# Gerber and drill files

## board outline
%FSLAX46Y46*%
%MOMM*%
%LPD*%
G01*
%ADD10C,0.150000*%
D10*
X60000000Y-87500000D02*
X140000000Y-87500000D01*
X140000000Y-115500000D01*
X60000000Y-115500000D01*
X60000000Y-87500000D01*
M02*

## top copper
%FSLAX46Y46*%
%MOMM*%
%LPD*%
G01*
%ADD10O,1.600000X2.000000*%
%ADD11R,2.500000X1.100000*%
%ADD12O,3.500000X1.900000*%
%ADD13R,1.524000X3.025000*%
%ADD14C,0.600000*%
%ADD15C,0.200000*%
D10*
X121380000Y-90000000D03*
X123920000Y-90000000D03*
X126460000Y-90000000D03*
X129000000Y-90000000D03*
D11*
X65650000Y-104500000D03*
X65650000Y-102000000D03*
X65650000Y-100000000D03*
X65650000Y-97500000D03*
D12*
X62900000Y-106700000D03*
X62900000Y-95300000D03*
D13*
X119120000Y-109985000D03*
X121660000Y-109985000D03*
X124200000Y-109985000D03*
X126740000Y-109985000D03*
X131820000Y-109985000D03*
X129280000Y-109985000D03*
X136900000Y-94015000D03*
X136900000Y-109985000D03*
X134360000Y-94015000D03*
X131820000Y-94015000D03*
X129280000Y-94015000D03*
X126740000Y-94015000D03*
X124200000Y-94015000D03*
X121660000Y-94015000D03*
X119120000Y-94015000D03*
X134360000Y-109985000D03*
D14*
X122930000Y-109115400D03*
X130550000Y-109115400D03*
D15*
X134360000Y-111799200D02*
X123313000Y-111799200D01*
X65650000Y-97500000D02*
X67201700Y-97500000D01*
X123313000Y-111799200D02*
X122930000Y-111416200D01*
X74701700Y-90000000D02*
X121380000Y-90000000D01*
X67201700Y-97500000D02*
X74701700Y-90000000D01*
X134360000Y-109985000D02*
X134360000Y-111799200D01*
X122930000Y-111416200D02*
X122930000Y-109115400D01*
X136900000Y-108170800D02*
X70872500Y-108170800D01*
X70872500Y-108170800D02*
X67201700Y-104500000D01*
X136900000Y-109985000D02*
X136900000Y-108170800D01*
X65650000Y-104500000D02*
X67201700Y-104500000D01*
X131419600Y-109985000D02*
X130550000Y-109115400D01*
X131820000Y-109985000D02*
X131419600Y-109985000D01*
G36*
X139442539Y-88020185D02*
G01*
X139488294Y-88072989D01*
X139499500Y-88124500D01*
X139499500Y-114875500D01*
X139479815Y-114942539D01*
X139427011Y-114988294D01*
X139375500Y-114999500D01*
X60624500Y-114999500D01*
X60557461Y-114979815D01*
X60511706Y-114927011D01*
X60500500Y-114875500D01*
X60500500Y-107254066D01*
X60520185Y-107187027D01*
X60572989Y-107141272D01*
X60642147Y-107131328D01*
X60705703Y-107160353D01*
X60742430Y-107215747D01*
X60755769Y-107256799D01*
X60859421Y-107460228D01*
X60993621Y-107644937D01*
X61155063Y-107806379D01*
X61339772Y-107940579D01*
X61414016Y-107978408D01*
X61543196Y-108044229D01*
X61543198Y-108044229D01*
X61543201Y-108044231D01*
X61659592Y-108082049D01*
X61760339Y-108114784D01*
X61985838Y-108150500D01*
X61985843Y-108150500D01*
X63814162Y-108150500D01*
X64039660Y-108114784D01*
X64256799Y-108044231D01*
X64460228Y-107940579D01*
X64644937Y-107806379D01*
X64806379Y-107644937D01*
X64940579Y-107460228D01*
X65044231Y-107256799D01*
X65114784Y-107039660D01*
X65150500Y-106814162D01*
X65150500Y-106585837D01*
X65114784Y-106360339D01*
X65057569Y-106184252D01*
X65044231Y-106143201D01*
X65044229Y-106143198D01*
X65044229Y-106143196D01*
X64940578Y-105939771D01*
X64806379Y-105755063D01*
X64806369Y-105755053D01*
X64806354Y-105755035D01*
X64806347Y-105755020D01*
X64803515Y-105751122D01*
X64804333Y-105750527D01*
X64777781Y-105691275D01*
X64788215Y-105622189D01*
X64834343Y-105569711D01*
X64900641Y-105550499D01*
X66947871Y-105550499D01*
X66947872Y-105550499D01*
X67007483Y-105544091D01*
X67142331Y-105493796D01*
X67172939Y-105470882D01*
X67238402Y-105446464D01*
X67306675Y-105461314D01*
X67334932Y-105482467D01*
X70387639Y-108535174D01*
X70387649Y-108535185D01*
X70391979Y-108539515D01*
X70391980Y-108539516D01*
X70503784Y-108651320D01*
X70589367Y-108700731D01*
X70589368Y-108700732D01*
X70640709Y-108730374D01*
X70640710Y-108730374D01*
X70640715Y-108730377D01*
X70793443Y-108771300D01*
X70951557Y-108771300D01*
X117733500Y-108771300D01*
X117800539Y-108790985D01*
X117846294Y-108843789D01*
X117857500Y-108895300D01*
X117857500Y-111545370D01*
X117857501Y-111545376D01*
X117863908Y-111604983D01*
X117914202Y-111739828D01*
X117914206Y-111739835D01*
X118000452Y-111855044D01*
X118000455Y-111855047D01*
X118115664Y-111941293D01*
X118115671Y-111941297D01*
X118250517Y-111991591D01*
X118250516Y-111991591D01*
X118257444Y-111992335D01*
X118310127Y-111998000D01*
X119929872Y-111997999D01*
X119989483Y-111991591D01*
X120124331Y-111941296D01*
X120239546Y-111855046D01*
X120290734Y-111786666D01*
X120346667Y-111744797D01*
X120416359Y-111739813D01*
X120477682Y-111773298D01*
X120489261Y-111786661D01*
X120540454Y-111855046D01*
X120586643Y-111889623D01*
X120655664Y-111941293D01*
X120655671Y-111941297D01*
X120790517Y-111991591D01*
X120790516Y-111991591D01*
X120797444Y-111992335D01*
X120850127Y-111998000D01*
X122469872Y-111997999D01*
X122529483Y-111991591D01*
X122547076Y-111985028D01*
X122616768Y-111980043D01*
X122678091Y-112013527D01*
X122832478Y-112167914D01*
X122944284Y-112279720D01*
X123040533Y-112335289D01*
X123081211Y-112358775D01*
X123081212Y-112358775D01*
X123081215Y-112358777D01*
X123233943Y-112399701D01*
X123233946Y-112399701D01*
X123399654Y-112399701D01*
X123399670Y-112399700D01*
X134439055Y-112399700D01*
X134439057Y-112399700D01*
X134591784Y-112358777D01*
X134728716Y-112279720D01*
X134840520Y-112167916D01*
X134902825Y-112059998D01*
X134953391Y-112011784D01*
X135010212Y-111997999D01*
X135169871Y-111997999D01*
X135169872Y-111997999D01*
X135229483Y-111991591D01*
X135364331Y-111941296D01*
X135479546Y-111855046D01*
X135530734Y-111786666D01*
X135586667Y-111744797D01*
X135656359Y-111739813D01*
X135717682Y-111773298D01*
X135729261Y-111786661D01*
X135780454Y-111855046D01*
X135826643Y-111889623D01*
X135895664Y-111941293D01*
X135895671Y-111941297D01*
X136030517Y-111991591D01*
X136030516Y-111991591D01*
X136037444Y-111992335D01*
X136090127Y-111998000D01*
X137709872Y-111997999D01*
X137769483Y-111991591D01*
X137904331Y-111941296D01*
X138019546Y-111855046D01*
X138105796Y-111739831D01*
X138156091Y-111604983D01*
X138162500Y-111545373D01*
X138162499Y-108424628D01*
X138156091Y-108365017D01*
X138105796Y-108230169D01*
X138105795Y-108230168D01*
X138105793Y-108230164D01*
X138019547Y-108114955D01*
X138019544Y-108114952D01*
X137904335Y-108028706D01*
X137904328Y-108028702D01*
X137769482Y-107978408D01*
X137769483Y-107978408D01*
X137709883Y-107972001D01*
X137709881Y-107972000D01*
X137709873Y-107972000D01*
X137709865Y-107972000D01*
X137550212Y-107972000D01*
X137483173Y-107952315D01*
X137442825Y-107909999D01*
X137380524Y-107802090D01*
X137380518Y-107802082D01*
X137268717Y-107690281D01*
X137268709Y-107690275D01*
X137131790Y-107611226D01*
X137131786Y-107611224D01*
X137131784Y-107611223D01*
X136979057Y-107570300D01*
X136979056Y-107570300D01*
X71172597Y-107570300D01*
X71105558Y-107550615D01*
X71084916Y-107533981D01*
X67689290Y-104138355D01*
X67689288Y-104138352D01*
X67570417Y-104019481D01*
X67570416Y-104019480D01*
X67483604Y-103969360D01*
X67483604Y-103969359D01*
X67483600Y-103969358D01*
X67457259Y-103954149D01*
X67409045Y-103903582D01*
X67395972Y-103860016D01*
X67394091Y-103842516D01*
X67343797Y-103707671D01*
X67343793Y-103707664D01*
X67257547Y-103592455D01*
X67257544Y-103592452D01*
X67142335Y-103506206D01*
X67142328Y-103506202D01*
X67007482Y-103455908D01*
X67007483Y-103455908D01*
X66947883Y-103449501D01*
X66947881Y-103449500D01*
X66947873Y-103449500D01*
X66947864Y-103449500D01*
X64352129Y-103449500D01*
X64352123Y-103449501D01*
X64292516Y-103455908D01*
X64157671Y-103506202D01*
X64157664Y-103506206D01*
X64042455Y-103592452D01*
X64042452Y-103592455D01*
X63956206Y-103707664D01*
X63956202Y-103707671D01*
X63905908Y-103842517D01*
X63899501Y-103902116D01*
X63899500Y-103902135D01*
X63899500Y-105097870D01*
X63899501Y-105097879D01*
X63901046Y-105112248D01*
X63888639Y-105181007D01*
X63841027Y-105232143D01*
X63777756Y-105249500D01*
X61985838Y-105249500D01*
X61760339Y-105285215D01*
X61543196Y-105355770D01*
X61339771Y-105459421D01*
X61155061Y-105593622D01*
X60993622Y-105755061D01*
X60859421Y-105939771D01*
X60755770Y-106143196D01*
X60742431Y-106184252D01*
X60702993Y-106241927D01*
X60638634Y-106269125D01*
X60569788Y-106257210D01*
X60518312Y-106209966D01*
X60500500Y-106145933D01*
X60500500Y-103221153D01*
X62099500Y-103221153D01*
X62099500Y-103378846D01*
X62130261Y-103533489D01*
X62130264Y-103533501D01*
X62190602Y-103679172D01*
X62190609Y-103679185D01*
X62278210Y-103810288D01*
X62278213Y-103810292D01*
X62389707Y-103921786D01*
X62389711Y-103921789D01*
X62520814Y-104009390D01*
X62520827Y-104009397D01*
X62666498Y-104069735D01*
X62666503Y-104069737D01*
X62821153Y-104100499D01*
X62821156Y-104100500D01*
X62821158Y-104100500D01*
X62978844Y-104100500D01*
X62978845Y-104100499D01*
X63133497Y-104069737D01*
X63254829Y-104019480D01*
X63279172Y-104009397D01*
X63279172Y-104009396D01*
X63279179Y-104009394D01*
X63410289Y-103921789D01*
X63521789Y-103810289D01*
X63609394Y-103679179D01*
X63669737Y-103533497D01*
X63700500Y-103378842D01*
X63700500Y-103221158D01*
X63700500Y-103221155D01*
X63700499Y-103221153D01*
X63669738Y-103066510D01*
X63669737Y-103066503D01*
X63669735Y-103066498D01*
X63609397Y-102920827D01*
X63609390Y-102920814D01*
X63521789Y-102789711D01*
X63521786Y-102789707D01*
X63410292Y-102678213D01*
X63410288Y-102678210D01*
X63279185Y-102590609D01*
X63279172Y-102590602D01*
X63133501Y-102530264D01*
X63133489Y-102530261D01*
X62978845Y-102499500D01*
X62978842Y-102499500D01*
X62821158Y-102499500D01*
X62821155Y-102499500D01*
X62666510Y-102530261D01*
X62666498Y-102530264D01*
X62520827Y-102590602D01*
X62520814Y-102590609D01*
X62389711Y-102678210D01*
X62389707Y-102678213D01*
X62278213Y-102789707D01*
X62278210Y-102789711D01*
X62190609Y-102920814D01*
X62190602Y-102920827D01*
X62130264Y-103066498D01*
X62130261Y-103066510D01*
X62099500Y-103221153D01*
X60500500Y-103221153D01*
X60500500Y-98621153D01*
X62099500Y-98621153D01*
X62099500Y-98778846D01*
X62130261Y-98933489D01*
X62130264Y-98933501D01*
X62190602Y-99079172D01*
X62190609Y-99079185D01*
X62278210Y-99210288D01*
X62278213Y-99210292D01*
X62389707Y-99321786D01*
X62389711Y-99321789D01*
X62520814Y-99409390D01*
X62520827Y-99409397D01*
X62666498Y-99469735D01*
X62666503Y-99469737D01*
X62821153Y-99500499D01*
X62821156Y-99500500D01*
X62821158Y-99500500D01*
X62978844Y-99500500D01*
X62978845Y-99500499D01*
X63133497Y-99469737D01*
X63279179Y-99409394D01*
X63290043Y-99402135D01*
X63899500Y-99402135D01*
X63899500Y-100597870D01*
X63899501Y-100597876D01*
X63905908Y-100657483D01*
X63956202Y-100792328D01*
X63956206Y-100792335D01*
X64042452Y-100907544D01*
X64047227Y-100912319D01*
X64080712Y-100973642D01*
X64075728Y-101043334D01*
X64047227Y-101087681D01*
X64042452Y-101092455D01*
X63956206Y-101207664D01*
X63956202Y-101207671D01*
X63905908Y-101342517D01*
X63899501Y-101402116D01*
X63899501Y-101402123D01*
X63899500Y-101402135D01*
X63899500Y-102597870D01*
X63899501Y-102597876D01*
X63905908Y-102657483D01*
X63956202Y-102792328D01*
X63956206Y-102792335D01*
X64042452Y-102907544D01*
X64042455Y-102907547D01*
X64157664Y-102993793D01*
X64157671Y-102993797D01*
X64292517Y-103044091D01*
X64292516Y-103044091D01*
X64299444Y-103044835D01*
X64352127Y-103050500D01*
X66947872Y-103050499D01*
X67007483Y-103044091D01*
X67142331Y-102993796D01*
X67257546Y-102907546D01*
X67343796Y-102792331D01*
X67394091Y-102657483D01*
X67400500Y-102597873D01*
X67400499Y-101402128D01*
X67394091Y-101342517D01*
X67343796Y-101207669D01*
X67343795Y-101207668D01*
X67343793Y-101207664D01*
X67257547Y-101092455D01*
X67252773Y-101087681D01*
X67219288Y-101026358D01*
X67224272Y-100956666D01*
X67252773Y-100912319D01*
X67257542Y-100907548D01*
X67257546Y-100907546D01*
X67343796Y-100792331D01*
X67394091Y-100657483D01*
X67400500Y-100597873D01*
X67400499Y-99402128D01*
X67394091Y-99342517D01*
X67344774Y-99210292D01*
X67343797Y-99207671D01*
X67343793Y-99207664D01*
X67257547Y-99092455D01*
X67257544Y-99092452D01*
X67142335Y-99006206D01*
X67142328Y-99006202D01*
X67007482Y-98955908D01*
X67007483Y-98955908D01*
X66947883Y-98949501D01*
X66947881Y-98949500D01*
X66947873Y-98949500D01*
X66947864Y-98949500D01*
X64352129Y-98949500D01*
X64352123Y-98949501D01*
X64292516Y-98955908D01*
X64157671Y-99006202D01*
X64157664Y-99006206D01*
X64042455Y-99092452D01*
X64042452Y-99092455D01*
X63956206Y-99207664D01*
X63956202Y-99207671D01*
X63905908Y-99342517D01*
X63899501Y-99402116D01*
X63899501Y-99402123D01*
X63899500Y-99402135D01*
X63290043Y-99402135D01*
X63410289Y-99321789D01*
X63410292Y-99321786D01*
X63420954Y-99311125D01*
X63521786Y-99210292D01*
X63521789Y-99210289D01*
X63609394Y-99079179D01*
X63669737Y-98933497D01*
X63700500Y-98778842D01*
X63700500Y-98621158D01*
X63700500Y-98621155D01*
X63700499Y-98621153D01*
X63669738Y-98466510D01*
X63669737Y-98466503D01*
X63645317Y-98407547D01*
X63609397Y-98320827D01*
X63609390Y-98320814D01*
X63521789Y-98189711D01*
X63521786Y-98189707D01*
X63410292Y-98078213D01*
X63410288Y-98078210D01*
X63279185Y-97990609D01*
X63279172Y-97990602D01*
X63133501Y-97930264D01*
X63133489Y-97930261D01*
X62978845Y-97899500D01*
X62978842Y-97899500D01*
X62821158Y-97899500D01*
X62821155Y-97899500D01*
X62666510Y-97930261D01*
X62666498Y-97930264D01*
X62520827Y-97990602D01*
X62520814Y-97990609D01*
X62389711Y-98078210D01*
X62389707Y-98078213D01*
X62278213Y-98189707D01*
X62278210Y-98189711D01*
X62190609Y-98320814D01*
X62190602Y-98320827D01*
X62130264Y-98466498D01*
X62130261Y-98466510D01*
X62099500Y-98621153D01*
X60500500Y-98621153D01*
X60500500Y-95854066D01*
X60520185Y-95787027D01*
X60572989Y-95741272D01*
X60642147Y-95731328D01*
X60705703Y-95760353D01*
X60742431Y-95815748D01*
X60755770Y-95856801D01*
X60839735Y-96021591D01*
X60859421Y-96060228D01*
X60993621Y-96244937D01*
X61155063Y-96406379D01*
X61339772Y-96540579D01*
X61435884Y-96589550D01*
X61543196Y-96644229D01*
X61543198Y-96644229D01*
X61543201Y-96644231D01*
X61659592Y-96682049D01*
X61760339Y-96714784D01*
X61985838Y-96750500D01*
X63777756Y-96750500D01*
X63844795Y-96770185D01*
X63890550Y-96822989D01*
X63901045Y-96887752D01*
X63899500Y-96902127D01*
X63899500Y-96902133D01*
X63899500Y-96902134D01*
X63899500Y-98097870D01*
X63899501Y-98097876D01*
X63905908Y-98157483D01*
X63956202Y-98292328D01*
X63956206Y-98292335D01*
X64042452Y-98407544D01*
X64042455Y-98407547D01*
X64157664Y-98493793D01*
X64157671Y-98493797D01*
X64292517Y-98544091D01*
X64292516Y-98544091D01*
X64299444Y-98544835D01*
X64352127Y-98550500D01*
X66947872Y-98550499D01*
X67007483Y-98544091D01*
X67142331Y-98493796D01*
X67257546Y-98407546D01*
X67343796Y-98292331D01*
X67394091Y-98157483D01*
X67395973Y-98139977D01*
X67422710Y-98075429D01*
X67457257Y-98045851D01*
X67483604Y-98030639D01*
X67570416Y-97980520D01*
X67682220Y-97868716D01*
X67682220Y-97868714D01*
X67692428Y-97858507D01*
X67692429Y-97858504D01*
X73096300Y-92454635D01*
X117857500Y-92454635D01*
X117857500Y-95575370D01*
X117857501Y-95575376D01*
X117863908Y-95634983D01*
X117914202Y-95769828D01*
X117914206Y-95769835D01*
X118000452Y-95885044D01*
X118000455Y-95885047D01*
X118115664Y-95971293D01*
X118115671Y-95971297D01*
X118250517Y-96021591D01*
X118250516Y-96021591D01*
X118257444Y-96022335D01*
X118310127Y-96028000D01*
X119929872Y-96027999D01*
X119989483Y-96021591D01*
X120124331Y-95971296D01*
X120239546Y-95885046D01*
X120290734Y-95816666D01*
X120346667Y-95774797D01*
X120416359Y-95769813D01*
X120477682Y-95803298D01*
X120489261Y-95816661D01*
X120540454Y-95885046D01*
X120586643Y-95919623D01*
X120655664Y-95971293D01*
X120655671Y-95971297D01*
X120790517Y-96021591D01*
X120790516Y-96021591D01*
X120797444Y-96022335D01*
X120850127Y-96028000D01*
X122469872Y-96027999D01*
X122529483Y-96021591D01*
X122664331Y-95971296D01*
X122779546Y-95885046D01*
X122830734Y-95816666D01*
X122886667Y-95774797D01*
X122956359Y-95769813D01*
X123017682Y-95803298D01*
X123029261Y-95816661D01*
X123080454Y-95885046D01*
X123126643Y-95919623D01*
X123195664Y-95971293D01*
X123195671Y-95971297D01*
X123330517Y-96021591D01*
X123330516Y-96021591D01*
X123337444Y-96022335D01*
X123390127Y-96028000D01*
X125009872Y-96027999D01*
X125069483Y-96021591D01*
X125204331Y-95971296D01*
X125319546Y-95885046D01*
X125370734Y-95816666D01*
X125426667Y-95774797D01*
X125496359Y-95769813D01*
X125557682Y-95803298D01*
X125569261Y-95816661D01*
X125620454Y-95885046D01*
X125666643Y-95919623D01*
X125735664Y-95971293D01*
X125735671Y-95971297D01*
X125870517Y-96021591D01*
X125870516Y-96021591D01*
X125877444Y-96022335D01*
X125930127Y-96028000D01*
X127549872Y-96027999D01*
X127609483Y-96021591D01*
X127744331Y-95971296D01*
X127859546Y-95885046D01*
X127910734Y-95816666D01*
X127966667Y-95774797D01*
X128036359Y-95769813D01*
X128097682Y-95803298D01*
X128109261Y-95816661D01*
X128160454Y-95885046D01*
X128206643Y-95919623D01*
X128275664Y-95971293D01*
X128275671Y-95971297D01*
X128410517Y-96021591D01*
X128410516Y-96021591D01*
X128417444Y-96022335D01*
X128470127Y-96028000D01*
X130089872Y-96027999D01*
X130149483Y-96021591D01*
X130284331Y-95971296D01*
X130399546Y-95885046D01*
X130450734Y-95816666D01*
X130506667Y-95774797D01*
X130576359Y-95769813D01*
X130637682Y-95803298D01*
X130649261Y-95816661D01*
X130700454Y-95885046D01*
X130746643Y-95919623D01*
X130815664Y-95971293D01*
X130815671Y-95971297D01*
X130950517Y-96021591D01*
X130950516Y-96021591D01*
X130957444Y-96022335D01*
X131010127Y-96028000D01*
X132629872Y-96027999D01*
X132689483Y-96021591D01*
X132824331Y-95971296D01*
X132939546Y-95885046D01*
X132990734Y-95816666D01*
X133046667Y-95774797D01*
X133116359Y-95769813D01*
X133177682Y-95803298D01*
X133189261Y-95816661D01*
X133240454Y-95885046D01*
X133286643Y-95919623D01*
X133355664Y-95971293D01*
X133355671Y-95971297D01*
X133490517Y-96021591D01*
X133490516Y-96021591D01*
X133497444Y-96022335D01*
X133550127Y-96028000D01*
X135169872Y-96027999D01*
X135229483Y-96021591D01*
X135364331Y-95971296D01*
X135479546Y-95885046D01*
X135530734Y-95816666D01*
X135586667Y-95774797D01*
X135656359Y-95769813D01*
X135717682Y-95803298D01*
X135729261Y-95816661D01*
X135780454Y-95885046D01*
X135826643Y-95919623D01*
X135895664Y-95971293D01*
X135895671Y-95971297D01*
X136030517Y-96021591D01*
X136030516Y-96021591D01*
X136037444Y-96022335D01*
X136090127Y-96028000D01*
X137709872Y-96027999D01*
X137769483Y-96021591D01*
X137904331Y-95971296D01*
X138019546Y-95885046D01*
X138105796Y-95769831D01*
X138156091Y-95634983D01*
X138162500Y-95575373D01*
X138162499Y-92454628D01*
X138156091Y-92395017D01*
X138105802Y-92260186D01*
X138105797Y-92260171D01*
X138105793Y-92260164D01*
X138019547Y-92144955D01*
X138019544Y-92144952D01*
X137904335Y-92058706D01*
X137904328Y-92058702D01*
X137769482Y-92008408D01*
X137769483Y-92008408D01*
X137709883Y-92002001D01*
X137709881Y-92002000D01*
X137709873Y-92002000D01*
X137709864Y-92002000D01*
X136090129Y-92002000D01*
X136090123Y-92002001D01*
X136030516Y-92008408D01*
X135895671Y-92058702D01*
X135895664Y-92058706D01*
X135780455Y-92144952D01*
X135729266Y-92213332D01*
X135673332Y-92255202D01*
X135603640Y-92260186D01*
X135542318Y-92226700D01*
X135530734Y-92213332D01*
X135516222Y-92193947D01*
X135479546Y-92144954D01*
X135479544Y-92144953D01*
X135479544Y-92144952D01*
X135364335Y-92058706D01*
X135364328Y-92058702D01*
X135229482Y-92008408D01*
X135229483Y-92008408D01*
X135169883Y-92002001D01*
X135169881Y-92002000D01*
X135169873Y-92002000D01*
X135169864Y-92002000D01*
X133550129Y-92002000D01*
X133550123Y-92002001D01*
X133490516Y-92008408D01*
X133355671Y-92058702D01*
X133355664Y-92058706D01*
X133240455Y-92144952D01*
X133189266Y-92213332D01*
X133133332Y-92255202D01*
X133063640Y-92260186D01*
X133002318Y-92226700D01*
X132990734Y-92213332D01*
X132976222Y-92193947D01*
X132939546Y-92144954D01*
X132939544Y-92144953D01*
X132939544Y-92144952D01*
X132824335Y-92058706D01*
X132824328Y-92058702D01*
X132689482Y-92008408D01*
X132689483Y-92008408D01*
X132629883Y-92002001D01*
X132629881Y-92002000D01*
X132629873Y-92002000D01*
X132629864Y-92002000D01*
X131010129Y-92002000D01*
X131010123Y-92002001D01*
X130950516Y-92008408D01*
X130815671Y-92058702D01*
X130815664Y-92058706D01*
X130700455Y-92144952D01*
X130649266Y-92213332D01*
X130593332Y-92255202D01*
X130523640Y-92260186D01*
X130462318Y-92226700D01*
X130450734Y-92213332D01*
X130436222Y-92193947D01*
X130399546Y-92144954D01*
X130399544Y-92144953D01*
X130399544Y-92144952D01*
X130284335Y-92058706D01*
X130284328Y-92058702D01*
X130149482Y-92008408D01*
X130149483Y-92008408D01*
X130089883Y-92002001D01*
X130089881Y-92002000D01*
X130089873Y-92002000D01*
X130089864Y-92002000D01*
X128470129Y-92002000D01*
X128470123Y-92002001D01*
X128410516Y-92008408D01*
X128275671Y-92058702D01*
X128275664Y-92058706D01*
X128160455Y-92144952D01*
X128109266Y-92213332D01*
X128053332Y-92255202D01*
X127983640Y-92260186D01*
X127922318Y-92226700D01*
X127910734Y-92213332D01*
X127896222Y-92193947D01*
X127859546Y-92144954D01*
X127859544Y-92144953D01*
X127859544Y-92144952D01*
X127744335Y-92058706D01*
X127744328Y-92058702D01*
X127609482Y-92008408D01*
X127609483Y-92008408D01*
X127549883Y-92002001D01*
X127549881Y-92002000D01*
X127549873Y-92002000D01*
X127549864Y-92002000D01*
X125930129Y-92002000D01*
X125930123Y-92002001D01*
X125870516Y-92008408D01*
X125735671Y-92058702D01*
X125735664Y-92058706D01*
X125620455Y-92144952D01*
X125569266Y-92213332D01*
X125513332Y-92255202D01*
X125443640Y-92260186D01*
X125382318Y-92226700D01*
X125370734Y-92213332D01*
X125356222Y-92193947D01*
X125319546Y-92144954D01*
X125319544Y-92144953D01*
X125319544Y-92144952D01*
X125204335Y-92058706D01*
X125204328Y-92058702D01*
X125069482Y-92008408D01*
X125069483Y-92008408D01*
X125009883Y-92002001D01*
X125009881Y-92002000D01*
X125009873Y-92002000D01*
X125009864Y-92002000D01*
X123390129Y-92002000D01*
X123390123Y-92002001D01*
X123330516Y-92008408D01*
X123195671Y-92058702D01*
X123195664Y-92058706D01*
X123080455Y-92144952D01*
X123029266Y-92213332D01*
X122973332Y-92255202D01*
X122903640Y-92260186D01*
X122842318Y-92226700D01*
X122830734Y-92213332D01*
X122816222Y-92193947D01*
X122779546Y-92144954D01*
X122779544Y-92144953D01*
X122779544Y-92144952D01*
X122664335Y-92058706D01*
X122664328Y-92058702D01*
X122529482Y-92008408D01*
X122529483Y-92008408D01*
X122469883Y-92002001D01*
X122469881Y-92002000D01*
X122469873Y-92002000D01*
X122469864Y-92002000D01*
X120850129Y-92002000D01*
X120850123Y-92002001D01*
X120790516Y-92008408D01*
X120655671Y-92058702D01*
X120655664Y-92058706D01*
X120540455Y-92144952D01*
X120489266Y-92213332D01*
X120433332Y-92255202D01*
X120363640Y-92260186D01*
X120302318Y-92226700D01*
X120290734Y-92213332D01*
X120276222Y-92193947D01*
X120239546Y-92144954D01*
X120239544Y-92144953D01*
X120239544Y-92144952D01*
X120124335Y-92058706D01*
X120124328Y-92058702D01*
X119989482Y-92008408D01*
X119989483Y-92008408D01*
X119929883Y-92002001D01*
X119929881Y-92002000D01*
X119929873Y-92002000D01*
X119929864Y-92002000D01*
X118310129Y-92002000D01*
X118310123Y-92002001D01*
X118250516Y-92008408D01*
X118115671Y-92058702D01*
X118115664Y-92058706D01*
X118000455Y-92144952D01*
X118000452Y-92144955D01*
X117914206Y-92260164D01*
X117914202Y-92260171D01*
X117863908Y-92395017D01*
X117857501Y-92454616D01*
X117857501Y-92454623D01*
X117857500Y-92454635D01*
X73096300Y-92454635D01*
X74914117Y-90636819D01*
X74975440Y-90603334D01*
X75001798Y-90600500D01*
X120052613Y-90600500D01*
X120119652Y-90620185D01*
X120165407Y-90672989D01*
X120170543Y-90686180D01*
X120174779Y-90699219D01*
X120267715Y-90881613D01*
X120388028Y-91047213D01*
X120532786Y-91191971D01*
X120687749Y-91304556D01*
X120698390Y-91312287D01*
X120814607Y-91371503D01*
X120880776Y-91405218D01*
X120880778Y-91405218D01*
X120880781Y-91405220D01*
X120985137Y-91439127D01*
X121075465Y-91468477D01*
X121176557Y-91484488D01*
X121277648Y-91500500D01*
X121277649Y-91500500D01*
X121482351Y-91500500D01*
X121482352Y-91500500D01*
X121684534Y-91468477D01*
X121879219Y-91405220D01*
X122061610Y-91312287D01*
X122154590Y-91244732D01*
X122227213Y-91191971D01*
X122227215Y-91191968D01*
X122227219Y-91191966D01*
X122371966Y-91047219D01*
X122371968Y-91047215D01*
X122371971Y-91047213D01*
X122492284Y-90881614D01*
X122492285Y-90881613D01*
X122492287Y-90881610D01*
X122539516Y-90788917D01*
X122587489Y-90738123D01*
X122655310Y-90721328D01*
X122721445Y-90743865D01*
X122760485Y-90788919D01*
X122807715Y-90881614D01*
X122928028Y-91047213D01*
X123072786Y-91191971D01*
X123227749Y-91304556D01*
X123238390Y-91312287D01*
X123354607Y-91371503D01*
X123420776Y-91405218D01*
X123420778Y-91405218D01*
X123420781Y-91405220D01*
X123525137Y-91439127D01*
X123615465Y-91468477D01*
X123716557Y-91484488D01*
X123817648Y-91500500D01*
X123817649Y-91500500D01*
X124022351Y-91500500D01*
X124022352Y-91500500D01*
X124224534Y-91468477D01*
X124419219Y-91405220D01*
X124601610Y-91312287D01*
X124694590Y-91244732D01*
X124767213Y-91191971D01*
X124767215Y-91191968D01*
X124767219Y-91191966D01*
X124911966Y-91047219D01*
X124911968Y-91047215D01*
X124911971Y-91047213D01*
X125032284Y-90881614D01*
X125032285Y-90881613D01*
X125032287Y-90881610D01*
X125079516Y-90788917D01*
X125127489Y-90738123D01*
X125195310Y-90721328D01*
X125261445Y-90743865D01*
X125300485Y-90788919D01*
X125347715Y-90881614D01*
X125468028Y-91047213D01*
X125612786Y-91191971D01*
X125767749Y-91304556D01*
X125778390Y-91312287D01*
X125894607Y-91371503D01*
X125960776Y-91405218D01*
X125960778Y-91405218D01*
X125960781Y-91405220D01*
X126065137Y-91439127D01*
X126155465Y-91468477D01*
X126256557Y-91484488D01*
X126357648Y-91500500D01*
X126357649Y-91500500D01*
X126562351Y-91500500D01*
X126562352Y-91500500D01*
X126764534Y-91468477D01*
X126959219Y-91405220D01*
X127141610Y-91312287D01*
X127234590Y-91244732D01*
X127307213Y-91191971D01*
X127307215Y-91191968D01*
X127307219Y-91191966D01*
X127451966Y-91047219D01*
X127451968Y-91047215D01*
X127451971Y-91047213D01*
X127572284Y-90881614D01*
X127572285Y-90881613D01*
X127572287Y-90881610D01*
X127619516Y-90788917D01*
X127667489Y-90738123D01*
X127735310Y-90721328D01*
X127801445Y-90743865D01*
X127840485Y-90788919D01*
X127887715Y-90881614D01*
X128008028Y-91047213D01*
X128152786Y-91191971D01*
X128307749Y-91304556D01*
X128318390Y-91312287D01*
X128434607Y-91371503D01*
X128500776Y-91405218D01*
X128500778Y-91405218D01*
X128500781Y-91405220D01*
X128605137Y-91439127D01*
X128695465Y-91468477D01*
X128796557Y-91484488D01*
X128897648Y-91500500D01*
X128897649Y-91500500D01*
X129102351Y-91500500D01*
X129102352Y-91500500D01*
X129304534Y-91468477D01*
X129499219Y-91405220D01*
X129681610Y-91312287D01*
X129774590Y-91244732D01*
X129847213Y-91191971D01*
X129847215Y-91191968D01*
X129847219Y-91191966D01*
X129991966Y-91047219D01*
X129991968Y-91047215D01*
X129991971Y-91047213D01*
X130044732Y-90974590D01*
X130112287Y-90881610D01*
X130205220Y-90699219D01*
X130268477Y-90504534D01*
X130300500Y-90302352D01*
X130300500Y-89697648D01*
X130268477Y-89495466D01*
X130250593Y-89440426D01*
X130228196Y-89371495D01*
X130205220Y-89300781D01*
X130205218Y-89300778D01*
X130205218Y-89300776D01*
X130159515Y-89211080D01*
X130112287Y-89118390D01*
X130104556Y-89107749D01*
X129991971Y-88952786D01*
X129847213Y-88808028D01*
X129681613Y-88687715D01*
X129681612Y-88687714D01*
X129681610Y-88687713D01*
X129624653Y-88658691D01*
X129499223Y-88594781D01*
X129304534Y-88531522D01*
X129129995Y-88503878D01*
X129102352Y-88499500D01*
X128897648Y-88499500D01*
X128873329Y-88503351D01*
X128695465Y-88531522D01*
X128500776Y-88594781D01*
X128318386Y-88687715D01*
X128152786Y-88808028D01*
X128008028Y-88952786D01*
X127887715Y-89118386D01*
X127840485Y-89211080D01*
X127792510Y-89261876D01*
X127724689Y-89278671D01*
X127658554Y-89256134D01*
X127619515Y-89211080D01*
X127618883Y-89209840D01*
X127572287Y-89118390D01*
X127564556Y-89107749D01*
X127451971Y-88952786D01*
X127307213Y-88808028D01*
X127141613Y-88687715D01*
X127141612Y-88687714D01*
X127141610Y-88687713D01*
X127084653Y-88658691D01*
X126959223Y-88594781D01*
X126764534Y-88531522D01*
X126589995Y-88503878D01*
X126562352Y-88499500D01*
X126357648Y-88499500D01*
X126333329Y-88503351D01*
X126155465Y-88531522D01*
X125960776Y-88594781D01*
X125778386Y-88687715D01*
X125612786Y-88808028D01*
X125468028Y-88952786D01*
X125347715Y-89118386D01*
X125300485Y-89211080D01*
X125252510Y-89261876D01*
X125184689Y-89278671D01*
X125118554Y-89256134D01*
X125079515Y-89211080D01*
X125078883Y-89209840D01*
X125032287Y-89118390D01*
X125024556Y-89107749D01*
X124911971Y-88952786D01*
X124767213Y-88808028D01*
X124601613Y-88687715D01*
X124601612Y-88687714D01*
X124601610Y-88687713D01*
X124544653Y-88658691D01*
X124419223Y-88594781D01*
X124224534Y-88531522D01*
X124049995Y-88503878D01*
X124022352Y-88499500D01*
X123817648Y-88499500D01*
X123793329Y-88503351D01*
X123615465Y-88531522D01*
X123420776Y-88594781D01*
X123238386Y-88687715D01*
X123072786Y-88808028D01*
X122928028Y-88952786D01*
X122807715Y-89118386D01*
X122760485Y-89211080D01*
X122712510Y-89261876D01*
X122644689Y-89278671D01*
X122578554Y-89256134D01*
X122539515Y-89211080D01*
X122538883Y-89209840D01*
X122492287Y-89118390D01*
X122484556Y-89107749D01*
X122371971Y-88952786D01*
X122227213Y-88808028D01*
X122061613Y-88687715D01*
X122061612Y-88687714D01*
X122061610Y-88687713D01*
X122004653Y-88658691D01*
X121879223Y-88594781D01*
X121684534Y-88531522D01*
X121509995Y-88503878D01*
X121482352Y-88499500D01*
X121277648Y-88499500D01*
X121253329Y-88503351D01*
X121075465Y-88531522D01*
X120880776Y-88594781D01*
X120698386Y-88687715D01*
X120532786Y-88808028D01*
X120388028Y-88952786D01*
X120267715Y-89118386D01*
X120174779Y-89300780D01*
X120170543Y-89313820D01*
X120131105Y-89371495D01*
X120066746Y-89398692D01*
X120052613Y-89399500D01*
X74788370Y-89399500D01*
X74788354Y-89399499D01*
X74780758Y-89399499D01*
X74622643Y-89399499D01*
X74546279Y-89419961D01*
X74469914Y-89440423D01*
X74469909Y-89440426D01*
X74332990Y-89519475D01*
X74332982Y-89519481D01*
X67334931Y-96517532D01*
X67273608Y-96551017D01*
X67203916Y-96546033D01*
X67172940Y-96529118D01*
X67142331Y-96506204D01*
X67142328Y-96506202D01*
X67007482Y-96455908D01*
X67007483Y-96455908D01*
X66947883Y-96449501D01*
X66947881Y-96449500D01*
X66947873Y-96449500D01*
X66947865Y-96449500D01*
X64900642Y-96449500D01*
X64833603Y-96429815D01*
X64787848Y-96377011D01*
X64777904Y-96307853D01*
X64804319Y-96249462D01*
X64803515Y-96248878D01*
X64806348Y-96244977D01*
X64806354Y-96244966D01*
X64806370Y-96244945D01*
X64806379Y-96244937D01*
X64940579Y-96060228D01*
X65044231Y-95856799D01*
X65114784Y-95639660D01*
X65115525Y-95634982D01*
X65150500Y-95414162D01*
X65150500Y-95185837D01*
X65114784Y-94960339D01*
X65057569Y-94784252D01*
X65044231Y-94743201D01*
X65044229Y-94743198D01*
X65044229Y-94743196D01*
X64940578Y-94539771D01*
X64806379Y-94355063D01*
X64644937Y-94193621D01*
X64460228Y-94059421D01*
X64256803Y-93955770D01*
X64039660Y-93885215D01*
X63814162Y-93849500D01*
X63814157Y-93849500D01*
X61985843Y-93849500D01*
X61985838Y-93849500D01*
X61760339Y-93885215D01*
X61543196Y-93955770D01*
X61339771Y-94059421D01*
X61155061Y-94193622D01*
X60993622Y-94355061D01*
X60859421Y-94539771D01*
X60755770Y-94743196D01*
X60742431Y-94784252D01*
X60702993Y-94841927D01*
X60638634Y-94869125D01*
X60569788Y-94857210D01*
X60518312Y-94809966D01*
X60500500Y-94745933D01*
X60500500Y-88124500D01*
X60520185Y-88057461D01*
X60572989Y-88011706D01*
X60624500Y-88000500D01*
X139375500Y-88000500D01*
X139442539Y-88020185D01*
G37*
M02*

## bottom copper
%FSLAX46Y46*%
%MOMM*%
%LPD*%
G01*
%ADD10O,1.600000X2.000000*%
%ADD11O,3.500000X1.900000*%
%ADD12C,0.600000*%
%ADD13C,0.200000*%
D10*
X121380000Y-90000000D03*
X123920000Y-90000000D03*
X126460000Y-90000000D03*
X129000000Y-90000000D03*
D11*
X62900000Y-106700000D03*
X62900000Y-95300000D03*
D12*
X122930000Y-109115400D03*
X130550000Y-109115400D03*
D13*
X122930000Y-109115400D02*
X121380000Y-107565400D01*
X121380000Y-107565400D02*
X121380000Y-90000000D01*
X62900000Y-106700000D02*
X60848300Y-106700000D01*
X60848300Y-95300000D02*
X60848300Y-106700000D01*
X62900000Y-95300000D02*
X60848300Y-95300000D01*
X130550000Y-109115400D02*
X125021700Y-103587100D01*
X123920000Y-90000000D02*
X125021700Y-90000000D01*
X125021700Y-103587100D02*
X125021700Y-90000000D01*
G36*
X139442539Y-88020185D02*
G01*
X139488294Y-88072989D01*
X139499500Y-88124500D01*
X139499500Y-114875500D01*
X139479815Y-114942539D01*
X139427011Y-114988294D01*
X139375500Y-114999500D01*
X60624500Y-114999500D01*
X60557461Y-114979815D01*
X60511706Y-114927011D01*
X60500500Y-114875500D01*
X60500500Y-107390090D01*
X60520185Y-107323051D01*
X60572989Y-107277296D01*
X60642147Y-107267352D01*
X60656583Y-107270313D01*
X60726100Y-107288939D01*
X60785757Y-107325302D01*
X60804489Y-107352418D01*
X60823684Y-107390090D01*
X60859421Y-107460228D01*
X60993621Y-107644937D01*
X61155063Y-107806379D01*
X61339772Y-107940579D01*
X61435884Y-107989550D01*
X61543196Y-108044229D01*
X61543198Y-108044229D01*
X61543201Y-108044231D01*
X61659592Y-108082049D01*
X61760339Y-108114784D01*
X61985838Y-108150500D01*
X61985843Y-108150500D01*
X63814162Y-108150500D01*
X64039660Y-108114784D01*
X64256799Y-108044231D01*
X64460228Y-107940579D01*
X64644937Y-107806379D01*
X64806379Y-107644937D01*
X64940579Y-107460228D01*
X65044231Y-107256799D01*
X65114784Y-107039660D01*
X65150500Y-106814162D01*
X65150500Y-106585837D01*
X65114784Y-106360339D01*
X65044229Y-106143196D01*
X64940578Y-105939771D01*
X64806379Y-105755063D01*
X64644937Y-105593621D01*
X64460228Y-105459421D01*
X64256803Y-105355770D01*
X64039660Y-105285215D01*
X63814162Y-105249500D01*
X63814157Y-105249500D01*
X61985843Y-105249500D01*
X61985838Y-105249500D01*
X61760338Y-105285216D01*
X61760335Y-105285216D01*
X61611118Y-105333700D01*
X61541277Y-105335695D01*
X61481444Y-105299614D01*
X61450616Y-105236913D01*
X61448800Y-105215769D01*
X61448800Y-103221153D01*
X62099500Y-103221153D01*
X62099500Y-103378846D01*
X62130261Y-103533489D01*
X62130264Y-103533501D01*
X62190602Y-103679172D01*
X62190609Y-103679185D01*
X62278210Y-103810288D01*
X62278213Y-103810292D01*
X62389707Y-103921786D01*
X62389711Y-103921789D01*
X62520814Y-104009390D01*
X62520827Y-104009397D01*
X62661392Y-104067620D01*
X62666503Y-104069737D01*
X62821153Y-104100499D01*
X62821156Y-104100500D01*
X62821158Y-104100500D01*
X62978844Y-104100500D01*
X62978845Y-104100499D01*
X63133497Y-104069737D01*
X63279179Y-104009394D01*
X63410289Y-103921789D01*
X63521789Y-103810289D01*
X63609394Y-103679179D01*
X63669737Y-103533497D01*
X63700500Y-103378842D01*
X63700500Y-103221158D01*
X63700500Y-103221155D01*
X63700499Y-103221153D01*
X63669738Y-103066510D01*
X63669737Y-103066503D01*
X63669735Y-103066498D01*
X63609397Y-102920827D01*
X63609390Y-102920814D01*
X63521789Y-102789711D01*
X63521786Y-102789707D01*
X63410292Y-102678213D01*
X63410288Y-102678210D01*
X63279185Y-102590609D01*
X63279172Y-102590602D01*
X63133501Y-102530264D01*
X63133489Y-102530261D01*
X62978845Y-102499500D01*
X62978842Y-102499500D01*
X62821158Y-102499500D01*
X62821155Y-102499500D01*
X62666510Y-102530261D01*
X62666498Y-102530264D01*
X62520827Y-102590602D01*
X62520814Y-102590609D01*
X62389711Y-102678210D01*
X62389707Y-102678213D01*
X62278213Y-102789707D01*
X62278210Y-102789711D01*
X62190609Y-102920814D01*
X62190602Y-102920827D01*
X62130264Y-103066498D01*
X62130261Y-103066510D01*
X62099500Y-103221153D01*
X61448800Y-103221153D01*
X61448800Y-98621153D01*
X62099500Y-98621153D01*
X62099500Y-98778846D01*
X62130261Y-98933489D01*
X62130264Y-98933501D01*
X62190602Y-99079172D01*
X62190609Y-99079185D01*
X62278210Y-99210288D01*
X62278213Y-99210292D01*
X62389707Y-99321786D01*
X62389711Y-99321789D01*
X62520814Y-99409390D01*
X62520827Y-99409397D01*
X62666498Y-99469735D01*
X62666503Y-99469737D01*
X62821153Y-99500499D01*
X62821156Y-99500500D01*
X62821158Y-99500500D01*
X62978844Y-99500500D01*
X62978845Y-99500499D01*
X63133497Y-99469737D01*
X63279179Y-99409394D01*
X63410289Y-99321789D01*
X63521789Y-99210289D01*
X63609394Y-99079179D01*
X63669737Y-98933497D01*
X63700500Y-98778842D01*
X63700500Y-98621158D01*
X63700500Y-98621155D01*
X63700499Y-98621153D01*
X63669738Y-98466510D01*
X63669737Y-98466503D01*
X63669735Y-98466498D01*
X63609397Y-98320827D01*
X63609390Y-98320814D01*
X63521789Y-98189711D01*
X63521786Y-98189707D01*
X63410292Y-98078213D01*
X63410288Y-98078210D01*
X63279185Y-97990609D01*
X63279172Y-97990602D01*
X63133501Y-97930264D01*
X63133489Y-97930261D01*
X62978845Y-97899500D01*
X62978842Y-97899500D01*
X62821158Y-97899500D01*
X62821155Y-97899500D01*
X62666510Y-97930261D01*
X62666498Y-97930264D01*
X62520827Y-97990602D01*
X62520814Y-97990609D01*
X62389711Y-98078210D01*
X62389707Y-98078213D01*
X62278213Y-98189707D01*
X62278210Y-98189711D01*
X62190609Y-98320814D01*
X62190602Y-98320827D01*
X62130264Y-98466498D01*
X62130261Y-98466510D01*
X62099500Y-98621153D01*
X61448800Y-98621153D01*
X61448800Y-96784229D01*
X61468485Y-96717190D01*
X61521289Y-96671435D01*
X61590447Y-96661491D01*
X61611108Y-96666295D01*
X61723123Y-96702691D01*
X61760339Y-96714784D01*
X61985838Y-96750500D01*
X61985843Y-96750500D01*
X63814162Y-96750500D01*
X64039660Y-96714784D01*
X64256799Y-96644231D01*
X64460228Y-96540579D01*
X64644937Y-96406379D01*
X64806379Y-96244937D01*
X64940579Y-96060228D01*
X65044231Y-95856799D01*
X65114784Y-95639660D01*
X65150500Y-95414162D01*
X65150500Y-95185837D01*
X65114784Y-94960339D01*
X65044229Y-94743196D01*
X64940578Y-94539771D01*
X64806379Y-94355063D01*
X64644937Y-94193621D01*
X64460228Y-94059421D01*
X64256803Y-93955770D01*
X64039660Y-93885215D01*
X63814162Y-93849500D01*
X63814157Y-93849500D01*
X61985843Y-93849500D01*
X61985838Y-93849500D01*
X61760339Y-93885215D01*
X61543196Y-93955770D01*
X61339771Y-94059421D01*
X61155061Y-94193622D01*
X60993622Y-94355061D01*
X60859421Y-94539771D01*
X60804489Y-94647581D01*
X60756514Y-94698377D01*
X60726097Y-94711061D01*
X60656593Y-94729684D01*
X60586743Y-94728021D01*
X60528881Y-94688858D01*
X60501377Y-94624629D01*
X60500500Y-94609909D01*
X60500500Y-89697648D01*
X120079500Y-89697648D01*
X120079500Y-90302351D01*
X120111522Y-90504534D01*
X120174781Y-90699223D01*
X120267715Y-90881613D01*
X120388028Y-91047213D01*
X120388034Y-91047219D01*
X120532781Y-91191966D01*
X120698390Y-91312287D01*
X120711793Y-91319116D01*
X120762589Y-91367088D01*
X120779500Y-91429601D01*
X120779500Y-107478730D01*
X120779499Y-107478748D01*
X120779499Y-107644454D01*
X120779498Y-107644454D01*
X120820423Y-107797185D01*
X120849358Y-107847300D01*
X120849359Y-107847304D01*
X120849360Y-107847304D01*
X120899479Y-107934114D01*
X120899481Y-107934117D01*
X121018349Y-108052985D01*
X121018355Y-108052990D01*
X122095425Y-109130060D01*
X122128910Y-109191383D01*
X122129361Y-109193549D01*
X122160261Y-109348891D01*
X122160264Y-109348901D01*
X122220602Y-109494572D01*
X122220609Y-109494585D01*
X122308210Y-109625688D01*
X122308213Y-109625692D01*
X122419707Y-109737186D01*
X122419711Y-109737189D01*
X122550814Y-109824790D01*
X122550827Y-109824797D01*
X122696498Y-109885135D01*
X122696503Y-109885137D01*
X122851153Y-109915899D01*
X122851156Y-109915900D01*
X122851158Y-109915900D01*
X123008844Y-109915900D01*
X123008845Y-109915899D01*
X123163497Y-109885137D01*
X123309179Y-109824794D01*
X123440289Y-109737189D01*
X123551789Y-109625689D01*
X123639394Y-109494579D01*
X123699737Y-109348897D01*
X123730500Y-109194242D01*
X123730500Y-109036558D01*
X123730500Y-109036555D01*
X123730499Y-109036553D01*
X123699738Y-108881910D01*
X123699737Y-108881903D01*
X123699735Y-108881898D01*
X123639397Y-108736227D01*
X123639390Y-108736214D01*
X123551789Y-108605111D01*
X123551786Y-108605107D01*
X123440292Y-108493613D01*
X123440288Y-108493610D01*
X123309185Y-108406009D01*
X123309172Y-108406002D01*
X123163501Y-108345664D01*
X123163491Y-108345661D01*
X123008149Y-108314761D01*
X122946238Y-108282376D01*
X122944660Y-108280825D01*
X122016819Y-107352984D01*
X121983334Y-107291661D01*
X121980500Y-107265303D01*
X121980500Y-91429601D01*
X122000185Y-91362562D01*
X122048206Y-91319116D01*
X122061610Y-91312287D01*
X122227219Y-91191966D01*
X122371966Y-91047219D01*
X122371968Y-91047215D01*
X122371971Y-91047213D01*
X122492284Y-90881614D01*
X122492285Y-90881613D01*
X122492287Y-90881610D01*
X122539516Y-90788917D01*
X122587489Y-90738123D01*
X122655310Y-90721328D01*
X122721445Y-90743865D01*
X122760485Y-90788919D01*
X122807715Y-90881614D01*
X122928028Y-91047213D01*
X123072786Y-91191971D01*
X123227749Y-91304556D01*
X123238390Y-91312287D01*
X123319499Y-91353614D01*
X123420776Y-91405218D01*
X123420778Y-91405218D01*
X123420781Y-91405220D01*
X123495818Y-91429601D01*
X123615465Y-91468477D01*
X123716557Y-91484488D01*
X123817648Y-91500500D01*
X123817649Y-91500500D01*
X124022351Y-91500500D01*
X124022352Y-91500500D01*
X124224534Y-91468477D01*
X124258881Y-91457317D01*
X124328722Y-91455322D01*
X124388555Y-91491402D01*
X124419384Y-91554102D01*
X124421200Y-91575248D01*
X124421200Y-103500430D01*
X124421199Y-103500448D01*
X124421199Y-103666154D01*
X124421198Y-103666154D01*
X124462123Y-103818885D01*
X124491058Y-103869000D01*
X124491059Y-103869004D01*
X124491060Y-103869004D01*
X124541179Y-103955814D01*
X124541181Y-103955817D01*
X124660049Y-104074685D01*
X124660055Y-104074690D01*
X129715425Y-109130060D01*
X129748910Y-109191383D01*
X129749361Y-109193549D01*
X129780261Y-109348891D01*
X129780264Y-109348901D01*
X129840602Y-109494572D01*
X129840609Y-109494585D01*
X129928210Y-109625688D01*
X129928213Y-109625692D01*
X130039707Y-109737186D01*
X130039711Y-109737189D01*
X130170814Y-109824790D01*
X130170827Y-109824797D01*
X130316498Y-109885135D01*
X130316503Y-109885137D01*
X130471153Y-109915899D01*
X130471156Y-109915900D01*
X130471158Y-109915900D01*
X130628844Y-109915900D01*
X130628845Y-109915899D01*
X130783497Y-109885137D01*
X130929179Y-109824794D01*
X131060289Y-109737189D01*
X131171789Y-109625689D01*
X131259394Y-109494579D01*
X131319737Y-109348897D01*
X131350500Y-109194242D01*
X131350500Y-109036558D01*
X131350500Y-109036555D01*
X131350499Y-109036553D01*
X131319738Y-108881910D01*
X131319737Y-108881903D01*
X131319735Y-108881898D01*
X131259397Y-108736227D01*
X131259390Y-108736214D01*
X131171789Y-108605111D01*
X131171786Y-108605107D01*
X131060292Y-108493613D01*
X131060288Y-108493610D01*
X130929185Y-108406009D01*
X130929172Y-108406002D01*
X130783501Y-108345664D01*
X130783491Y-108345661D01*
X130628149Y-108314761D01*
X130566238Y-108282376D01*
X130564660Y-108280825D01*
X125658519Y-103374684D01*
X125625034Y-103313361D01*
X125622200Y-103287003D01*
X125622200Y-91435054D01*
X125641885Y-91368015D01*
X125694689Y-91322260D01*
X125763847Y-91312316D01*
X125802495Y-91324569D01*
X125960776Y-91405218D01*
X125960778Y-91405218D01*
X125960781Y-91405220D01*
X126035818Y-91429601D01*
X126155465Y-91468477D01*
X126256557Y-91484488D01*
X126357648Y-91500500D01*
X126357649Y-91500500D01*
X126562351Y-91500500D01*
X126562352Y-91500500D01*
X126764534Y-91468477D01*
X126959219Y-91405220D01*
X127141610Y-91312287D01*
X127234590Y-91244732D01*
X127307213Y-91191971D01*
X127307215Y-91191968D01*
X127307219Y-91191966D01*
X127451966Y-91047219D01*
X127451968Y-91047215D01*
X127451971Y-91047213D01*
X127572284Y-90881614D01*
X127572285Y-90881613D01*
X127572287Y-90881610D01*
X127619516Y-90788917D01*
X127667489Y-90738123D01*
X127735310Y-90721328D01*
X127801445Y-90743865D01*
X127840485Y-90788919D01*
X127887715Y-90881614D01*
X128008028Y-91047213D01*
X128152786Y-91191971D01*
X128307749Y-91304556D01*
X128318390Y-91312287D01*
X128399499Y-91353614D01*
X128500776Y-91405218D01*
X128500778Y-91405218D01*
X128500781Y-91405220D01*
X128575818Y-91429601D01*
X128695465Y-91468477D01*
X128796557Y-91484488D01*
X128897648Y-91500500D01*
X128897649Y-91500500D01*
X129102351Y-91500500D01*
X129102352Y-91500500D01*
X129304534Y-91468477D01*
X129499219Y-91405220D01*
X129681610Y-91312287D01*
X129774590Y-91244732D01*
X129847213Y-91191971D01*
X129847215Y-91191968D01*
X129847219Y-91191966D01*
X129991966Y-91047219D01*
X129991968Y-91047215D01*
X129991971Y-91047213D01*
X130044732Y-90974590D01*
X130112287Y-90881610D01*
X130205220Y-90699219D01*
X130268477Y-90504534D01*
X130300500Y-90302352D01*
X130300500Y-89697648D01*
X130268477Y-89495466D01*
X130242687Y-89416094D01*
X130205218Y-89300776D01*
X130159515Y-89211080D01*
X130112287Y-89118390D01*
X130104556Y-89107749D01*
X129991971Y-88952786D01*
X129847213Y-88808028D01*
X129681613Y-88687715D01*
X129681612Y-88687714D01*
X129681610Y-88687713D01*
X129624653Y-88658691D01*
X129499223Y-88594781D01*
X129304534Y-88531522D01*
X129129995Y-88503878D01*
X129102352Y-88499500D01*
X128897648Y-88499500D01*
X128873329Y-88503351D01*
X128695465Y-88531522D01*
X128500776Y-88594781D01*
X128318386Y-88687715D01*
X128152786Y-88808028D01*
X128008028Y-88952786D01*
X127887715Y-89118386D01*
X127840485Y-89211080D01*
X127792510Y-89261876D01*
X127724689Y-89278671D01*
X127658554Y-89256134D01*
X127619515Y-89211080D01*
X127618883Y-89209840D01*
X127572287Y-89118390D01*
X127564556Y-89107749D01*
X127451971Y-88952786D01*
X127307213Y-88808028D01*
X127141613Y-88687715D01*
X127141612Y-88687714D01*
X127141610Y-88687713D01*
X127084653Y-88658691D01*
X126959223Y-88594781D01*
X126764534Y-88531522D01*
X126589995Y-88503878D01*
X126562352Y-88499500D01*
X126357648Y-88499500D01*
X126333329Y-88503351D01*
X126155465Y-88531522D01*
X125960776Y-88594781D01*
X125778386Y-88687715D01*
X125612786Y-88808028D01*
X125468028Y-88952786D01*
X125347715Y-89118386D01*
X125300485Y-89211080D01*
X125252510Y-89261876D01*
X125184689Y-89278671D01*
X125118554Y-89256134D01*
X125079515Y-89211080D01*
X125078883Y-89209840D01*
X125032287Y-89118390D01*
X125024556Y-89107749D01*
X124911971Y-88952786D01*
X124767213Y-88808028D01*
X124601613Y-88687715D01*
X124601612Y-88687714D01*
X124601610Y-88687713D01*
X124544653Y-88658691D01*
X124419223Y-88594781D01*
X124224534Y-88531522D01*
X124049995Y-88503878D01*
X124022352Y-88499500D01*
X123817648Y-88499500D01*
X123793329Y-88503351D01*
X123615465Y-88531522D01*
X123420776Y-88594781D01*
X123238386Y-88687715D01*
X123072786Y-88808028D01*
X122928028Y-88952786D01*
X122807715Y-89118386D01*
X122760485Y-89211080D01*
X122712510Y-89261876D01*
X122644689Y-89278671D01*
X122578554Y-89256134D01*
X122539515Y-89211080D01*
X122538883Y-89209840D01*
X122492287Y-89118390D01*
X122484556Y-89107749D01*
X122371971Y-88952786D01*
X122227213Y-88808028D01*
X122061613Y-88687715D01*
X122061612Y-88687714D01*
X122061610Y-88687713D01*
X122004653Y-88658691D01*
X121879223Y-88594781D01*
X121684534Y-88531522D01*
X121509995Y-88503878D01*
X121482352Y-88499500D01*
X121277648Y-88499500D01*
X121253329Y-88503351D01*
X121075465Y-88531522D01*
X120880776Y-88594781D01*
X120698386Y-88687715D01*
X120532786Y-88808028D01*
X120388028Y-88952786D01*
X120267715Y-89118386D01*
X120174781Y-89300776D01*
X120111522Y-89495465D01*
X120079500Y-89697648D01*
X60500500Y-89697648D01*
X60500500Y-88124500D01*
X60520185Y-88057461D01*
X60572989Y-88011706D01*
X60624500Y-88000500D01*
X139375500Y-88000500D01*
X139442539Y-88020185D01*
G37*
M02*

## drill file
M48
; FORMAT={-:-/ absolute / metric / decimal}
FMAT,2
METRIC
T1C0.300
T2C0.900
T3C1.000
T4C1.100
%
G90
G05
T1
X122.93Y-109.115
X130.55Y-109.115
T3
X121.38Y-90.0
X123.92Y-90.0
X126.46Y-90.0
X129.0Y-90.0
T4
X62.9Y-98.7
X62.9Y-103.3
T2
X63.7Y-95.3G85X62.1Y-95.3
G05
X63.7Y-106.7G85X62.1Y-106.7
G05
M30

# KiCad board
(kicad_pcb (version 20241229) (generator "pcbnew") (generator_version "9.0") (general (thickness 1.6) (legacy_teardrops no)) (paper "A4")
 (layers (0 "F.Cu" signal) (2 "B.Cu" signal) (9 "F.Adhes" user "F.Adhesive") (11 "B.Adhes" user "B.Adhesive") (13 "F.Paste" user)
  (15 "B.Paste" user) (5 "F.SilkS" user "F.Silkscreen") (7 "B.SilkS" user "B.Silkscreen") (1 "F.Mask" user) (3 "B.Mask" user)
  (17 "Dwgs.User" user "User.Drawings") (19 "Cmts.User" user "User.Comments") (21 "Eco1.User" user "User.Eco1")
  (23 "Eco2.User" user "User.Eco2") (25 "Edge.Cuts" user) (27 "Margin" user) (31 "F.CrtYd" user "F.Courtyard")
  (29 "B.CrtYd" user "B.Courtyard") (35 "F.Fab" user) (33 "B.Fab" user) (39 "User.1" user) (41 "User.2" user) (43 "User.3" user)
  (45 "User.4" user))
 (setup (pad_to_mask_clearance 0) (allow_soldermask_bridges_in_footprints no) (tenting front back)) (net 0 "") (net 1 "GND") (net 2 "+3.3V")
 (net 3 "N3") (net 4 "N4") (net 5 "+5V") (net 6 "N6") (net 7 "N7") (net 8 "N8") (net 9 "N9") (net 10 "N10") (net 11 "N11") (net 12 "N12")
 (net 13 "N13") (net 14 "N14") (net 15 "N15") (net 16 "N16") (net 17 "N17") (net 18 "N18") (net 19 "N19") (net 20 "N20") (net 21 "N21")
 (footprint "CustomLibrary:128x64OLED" (layer "F.Cu") (at 125 100.6)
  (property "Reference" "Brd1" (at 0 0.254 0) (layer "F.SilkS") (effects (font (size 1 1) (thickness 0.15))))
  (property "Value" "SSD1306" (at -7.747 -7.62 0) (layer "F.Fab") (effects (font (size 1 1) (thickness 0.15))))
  (pad "1" thru_hole oval (at -3.62 -10.6 90) (size 2 1.6) (drill 1) (layers "*.Cu" "*.Mask") (remove_unused_layers no) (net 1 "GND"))
  (pad "2" thru_hole oval (at -1.08 -10.6 90) (size 2 1.6) (drill 1) (layers "*.Cu" "*.Mask") (remove_unused_layers no) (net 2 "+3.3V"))
  (pad "3" thru_hole oval (at 1.46 -10.6 90) (size 2 1.6) (drill 1) (layers "*.Cu" "*.Mask") (remove_unused_layers no) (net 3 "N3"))
  (pad "4" thru_hole oval (at 4 -10.6 90) (size 2 1.6) (drill 1) (layers "*.Cu" "*.Mask") (remove_unused_layers no) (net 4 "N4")))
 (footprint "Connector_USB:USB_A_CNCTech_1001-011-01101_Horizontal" (layer "F.Cu") (at 56 101 180)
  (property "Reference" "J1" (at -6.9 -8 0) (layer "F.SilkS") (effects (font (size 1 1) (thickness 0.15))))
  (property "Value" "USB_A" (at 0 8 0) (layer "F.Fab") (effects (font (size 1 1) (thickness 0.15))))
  (pad "" np_thru_hole circle (at -6.9 -2.3 180) (size 1.1 1.1) (drill 1.1) (layers "*.Cu" "*.Mask"))
  (pad "" np_thru_hole circle (at -6.9 2.3 180) (size 1.1 1.1) (drill 1.1) (layers "*.Cu" "*.Mask"))
  (pad "1" smd rect (at -9.65 -3.5 180) (size 2.5 1.1) (layers "F.Cu" "F.Mask" "F.Paste") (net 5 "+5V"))
  (pad "2" smd rect (at -9.65 -1 180) (size 2.5 1.1) (layers "F.Cu" "F.Mask" "F.Paste") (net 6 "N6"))
  (pad "3" smd rect (at -9.65 1 180) (size 2.5 1.1) (layers "F.Cu" "F.Mask" "F.Paste") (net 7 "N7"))
  (pad "4" smd rect (at -9.65 3.5 180) (size 2.5 1.1) (layers "F.Cu" "F.Mask" "F.Paste") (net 1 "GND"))
  (pad "5" thru_hole oval (at -6.9 -5.7 180) (size 3.5 1.9) (drill oval 2.5 0.9) (layers "*.Cu" "*.Mask") (remove_unused_layers no)
   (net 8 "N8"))
  (pad "5" thru_hole oval (at -6.9 5.7 180) (size 3.5 1.9) (drill oval 2.5 0.9) (layers "*.Cu" "*.Mask") (remove_unused_layers no)
   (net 8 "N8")))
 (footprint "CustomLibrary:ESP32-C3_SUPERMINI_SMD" (layer "F.Cu") (at 127 102 -90)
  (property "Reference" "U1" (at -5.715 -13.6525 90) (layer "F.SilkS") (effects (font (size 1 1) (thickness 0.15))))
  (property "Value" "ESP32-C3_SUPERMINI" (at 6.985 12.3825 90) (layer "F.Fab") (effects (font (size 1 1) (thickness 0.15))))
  (pad "0" smd rect (at 7.985 7.88 270) (size 3.025 1.524) (layers "F.Cu" "F.Mask" "F.Paste") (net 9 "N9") (solder_mask_margin 0.102))
  (pad "1" smd rect (at 7.985 5.34 270) (size 3.025 1.524) (layers "F.Cu" "F.Mask" "F.Paste") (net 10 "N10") (solder_mask_margin 0.102))
  (pad "2" smd rect (at 7.985 2.8 270) (size 3.025 1.524) (layers "F.Cu" "F.Mask" "F.Paste") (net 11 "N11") (solder_mask_margin 0.102))
  (pad "3" smd rect (at 7.985 0.26 270) (size 3.025 1.524) (layers "F.Cu" "F.Mask" "F.Paste") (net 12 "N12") (solder_mask_margin 0.102))
  (pad "3.3" smd rect (at 7.985 -4.82 270) (size 3.025 1.524) (layers "F.Cu" "F.Mask" "F.Paste") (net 2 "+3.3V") (solder_mask_margin 0.102))
  (pad "4" smd rect (at 7.985 -2.28 270) (size 3.025 1.524) (layers "F.Cu" "F.Mask" "F.Paste") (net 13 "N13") (solder_mask_margin 0.102))
  (pad "5" smd rect (at -7.985 -9.9 270) (size 3.025 1.524) (layers "F.Cu" "F.Mask" "F.Paste") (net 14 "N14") (solder_mask_margin 0.102))
  (pad "5V" smd rect (at 7.985 -9.9 270) (size 3.025 1.524) (layers "F.Cu" "F.Mask" "F.Paste") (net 5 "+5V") (solder_mask_margin 0.102))
  (pad "6" smd rect (at -7.985 -7.36 270) (size 3.025 1.524) (layers "F.Cu" "F.Mask" "F.Paste") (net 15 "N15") (solder_mask_margin 0.102))
  (pad "7" smd rect (at -7.985 -4.82 270) (size 3.025 1.524) (layers "F.Cu" "F.Mask" "F.Paste") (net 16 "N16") (solder_mask_margin 0.102))
  (pad "8" smd rect (at -7.985 -2.28 270) (size 3.025 1.524) (layers "F.Cu" "F.Mask" "F.Paste") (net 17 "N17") (solder_mask_margin 0.102))
  (pad "9" smd rect (at -7.985 0.26 270) (size 3.025 1.524) (layers "F.Cu" "F.Mask" "F.Paste") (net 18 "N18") (solder_mask_margin 0.102))
  (pad "10" smd rect (at -7.985 2.8 270) (size 3.025 1.524) (layers "F.Cu" "F.Mask" "F.Paste") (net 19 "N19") (solder_mask_margin 0.102))
  (pad "20" smd rect (at -7.985 5.34 270) (size 3.025 1.524) (layers "F.Cu" "F.Mask" "F.Paste") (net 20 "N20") (solder_mask_margin 0.102))
  (pad "21" smd rect (at -7.985 7.88 270) (size 3.025 1.524) (layers "F.Cu" "F.Mask" "F.Paste") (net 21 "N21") (solder_mask_margin 0.102))
  (pad "G" smd rect (at 7.985 -7.36 270) (size 3.025 1.524) (layers "F.Cu" "F.Mask" "F.Paste") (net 1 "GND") (solder_mask_margin 0.102)))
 (gr_rect (start 60 87.5) (end 140 115.5) (stroke (width 0.15) (type default)) (fill no) (layer "Edge.Cuts"))
 (segment (start 134.36 111.7992) (end 123.313 111.7992) (width 0.2) (layer "F.Cu") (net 1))
 (segment (start 65.65 97.5) (end 67.2017 97.5) (width 0.2) (layer "F.Cu") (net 1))
 (segment (start 123.313 111.7992) (end 122.93 111.4162) (width 0.2) (layer "F.Cu") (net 1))
 (segment (start 74.7017 90) (end 121.38 90) (width 0.2) (layer "F.Cu") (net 1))
 (segment (start 67.2017 97.5) (end 74.7017 90) (width 0.2) (layer "F.Cu") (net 1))
 (segment (start 134.36 109.985) (end 134.36 111.7992) (width 0.2) (layer "F.Cu") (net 1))
 (segment (start 122.93 111.4162) (end 122.93 109.1154) (width 0.2) (layer "F.Cu") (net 1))
 (via (at 122.93 109.1154) (size 0.6) (drill 0.3) (layers "F.Cu" "B.Cu") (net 1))
 (segment (start 122.93 109.1154) (end 121.38 107.5654) (width 0.2) (layer "B.Cu") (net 1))
 (segment (start 121.38 107.5654) (end 121.38 90) (width 0.2) (layer "B.Cu") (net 1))
 (segment (start 136.9 108.1708) (end 70.8725 108.1708) (width 0.2) (layer "F.Cu") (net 5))
 (segment (start 70.8725 108.1708) (end 67.2017 104.5) (width 0.2) (layer "F.Cu") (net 5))
 (segment (start 136.9 109.985) (end 136.9 108.1708) (width 0.2) (layer "F.Cu") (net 5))
 (segment (start 65.65 104.5) (end 67.2017 104.5) (width 0.2) (layer "F.Cu") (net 5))
 (segment (start 62.9 106.7) (end 60.8483 106.7) (width 0.2) (layer "B.Cu") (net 8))
 (segment (start 60.8483 95.3) (end 60.8483 106.7) (width 0.2) (layer "B.Cu") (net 8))
 (segment (start 62.9 95.3) (end 60.8483 95.3) (width 0.2) (layer "B.Cu") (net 8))
 (segment (start 131.4196 109.985) (end 130.55 109.1154) (width 0.2) (layer "F.Cu") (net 2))
 (segment (start 131.82 109.985) (end 131.4196 109.985) (width 0.2) (layer "F.Cu") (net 2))
 (via (at 130.55 109.1154) (size 0.6) (drill 0.3) (layers "F.Cu" "B.Cu") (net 2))
 (segment (start 130.55 109.1154) (end 125.0217 103.5871) (width 0.2) (layer "B.Cu") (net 2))
 (segment (start 123.92 90) (end 125.0217 90) (width 0.2) (layer "B.Cu") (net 2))
 (segment (start 125.0217 103.5871) (end 125.0217 90) (width 0.2) (layer "B.Cu") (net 2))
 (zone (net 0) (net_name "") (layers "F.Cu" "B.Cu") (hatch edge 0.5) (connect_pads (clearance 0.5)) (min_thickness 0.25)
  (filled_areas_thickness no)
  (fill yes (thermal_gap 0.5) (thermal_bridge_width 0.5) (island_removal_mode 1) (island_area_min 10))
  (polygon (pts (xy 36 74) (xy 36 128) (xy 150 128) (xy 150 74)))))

